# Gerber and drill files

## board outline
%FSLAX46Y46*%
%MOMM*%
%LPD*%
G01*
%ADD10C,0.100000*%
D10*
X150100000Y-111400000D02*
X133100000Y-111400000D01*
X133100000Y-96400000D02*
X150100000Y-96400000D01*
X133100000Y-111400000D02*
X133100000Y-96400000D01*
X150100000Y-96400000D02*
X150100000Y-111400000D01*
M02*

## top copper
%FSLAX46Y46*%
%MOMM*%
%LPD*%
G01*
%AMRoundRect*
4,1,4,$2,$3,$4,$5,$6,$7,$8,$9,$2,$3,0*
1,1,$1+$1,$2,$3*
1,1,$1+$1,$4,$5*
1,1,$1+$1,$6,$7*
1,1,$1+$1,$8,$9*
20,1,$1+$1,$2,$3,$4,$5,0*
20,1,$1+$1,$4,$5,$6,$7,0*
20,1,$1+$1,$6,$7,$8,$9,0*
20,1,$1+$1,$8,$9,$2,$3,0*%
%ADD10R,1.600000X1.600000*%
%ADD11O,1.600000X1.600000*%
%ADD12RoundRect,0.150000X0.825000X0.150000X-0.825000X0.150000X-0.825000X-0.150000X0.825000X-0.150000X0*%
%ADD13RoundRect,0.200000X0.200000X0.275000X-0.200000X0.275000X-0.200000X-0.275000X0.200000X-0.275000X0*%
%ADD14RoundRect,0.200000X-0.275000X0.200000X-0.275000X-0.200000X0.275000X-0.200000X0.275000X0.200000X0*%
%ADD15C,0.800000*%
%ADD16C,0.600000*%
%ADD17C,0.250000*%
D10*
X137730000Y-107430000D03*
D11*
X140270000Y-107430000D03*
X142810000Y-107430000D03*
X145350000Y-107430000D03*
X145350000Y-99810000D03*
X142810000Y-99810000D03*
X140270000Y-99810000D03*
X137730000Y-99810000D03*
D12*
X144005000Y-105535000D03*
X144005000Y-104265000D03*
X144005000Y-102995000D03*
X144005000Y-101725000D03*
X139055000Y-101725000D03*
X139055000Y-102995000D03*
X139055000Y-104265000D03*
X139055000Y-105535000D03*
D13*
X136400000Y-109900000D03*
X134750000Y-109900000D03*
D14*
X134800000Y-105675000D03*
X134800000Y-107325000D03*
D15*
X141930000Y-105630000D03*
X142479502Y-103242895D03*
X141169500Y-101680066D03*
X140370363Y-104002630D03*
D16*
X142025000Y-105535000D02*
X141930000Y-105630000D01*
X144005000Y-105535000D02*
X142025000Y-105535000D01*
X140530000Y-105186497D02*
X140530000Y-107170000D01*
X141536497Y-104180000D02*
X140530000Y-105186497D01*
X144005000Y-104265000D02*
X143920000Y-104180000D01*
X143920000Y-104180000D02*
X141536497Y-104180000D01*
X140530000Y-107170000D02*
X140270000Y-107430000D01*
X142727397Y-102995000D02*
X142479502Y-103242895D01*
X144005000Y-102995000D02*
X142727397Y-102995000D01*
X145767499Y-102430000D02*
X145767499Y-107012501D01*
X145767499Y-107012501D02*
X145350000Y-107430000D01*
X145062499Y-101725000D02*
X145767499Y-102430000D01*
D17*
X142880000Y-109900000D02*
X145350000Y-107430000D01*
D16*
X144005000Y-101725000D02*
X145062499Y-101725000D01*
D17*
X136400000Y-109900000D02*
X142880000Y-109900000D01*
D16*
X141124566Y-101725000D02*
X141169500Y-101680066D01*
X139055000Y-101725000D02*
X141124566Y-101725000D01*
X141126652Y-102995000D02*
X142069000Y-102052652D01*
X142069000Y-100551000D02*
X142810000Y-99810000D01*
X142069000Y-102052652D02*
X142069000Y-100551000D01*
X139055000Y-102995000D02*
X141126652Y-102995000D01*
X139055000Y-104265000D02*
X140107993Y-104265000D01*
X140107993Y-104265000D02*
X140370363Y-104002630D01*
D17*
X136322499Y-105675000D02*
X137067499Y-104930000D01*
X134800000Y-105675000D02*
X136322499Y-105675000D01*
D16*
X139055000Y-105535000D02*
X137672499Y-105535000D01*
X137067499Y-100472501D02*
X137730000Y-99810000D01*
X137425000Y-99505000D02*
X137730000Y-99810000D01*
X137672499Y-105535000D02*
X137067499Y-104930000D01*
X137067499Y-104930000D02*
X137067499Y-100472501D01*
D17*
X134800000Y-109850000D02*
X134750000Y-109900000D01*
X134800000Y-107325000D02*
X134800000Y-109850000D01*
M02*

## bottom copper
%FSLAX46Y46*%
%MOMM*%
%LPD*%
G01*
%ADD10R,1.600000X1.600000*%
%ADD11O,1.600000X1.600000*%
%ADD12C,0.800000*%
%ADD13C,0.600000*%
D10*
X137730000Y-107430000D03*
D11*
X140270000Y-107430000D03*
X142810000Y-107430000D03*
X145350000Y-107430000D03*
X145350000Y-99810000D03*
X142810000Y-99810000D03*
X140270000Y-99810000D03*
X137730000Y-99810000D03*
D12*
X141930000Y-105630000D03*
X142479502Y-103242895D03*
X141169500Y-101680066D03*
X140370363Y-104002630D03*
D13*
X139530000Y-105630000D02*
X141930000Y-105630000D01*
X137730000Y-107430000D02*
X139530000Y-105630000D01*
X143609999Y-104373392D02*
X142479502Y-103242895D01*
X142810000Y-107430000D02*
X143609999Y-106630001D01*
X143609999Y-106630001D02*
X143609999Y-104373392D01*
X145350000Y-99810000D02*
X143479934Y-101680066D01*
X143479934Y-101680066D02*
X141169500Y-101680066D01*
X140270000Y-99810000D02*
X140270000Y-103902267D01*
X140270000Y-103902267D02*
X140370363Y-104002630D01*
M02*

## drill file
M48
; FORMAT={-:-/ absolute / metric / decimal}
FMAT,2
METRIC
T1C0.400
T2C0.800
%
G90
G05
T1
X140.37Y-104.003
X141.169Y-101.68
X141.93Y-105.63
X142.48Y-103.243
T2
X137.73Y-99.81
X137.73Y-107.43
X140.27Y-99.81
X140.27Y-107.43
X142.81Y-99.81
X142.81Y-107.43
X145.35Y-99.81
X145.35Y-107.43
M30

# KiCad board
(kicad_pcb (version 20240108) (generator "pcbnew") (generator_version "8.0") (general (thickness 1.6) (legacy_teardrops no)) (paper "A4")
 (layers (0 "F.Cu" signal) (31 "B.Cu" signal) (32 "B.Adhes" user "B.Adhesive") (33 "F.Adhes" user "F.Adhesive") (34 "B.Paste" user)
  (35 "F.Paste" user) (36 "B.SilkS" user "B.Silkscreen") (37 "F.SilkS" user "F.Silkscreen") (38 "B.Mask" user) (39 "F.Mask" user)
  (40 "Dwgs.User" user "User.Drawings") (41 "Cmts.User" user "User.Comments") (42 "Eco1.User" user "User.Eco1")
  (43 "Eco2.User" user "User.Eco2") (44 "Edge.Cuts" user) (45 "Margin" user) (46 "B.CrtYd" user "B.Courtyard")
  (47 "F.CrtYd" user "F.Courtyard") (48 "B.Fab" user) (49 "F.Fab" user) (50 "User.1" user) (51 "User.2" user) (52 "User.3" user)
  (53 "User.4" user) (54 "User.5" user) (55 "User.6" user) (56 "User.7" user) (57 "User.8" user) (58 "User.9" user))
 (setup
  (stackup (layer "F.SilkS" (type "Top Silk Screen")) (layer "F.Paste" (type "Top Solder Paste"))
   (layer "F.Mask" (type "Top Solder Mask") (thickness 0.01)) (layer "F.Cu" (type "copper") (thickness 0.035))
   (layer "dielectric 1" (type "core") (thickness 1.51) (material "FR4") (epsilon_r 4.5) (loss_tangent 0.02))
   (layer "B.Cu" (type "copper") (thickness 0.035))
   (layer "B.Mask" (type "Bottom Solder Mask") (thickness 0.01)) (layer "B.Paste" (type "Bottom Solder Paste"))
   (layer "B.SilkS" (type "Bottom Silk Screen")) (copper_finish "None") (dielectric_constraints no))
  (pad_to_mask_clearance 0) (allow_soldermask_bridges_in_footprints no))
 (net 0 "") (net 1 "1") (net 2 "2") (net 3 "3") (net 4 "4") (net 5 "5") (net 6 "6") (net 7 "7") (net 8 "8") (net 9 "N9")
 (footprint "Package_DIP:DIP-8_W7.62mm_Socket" (layer "F.Cu") (at 137.73 107.43 90)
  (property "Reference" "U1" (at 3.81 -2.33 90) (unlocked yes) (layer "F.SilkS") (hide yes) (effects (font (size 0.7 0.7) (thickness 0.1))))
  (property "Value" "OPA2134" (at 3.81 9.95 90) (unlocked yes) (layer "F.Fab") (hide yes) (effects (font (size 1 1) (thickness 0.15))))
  (pad "1" thru_hole rect (at 0 0 90) (size 1.6 1.6) (drill 0.8) (layers "*.Cu" "*.Mask") (remove_unused_layers no) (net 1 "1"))
  (pad "2" thru_hole oval (at 0 2.54 90) (size 1.6 1.6) (drill 0.8) (layers "*.Cu" "*.Mask") (remove_unused_layers no) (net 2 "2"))
  (pad "3" thru_hole oval (at 0 5.08 90) (size 1.6 1.6) (drill 0.8) (layers "*.Cu" "*.Mask") (remove_unused_layers no) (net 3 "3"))
  (pad "4" thru_hole oval (at 0 7.62 90) (size 1.6 1.6) (drill 0.8) (layers "*.Cu" "*.Mask") (remove_unused_layers no) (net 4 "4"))
  (pad "5" thru_hole oval (at 7.62 7.62 90) (size 1.6 1.6) (drill 0.8) (layers "*.Cu" "*.Mask") (remove_unused_layers no) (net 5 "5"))
  (pad "6" thru_hole oval (at 7.62 5.08 90) (size 1.6 1.6) (drill 0.8) (layers "*.Cu" "*.Mask") (remove_unused_layers no) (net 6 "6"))
  (pad "7" thru_hole oval (at 7.62 2.54 90) (size 1.6 1.6) (drill 0.8) (layers "*.Cu" "*.Mask") (remove_unused_layers no) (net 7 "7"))
  (pad "8" thru_hole oval (at 7.62 0 90) (size 1.6 1.6) (drill 0.8) (layers "*.Cu" "*.Mask") (remove_unused_layers no) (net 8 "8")))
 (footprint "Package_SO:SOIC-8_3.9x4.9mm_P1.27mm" (layer "F.Cu") (at 141.53 103.63 180)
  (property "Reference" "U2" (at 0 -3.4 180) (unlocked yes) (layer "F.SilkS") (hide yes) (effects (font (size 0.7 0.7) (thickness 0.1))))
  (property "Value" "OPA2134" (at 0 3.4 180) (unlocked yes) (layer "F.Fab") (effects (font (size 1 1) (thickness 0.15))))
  (pad "1" smd roundrect (at -2.475 -1.905 180) (size 1.95 0.6) (layers "F.Cu" "F.Paste" "F.Mask") (roundrect_rratio 0.25) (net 1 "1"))
  (pad "2" smd roundrect (at -2.475 -0.635 180) (size 1.95 0.6) (layers "F.Cu" "F.Paste" "F.Mask") (roundrect_rratio 0.25) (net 2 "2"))
  (pad "3" smd roundrect (at -2.475 0.635 180) (size 1.95 0.6) (layers "F.Cu" "F.Paste" "F.Mask") (roundrect_rratio 0.25) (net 3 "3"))
  (pad "4" smd roundrect (at -2.475 1.905 180) (size 1.95 0.6) (layers "F.Cu" "F.Paste" "F.Mask") (roundrect_rratio 0.25) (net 4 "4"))
  (pad "5" smd roundrect (at 2.475 1.905 180) (size 1.95 0.6) (layers "F.Cu" "F.Paste" "F.Mask") (roundrect_rratio 0.25) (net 5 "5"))
  (pad "6" smd roundrect (at 2.475 0.635 180) (size 1.95 0.6) (layers "F.Cu" "F.Paste" "F.Mask") (roundrect_rratio 0.25) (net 6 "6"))
  (pad "7" smd roundrect (at 2.475 -0.635 180) (size 1.95 0.6) (layers "F.Cu" "F.Paste" "F.Mask") (roundrect_rratio 0.25) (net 7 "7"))
  (pad "8" smd roundrect (at 2.475 -1.905 180) (size 1.95 0.6) (layers "F.Cu" "F.Paste" "F.Mask") (roundrect_rratio 0.25) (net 8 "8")))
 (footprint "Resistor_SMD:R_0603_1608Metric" (layer "F.Cu") (at 135.575 109.9 180)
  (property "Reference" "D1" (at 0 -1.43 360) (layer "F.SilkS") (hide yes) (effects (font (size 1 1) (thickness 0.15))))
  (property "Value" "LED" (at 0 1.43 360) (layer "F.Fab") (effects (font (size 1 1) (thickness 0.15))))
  (pad "1" smd roundrect (at -0.825 0 180) (size 0.8 0.95) (layers "F.Cu" "F.Paste" "F.Mask") (roundrect_rratio 0.25) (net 4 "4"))
  (pad "2" smd roundrect (at 0.825 0 180) (size 0.8 0.95) (layers "F.Cu" "F.Paste" "F.Mask") (roundrect_rratio 0.25) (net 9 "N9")))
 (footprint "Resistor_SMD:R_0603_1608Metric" (layer "F.Cu") (at 134.8 106.5 -90)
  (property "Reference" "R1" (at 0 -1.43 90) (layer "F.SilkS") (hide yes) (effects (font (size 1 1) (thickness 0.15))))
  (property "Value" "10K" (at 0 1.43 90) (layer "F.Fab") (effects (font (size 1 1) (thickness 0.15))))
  (pad "1" smd roundrect (at -0.825 0 270) (size 0.8 0.95) (layers "F.Cu" "F.Paste" "F.Mask") (roundrect_rratio 0.25) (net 8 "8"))
  (pad "2" smd roundrect (at 0.825 0 270) (size 0.8 0.95) (layers "F.Cu" "F.Paste" "F.Mask") (roundrect_rratio 0.25) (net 9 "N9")))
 (gr_line (start 150.1 111.4) (end 133.1 111.4) (stroke (width 0.1) (type default)) (layer "Edge.Cuts"))
 (gr_line (start 133.1 96.4) (end 150.1 96.4) (stroke (width 0.1) (type default)) (layer "Edge.Cuts"))
 (gr_line (start 133.1 111.4) (end 133.1 96.4) (stroke (width 0.1) (type default)) (layer "Edge.Cuts"))
 (gr_line (start 150.1 96.4) (end 150.1 111.4) (stroke (width 0.1) (type default)) (layer "Edge.Cuts"))
 (segment (start 142.025 105.535) (end 141.93 105.63) (width 0.6) (layer "F.Cu") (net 1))
 (segment (start 144.005 105.535) (end 142.025 105.535) (width 0.6) (layer "F.Cu") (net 1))
 (via (at 141.93 105.63) (size 0.8) (drill 0.4) (layers "F.Cu" "B.Cu") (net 1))
 (segment (start 139.53 105.63) (end 141.93 105.63) (width 0.6) (layer "B.Cu") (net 1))
 (segment (start 137.73 107.43) (end 139.53 105.63) (width 0.6) (layer "B.Cu") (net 1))
 (segment (start 140.53 105.186497) (end 140.53 107.17) (width 0.6) (layer "F.Cu") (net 2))
 (segment (start 141.536497 104.18) (end 140.53 105.186497) (width 0.6) (layer "F.Cu") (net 2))
 (segment (start 144.005 104.265) (end 143.92 104.18) (width 0.6) (layer "F.Cu") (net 2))
 (segment (start 143.92 104.18) (end 141.536497 104.18) (width 0.6) (layer "F.Cu") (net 2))
 (segment (start 140.53 107.17) (end 140.27 107.43) (width 0.6) (layer "F.Cu") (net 2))
 (segment (start 142.727397 102.995) (end 142.479502 103.242895) (width 0.6) (layer "F.Cu") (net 3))
 (segment (start 144.005 102.995) (end 142.727397 102.995) (width 0.6) (layer "F.Cu") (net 3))
 (via (at 142.479502 103.242895) (size 0.8) (drill 0.4) (layers "F.Cu" "B.Cu") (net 3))
 (segment (start 143.609999 104.373392) (end 142.479502 103.242895) (width 0.6) (layer "B.Cu") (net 3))
 (segment (start 142.81 107.43) (end 143.609999 106.630001) (width 0.6) (layer "B.Cu") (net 3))
 (segment (start 143.609999 106.630001) (end 143.609999 104.373392) (width 0.6) (layer "B.Cu") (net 3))
 (segment (start 145.767499 102.43) (end 145.767499 107.012501) (width 0.6) (layer "F.Cu") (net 4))
 (segment (start 145.767499 107.012501) (end 145.35 107.43) (width 0.6) (layer "F.Cu") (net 4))
 (segment (start 145.062499 101.725) (end 145.767499 102.43) (width 0.6) (layer "F.Cu") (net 4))
 (segment (start 142.88 109.9) (end 145.35 107.43) (width 0.25) (layer "F.Cu") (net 4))
 (segment (start 144.005 101.725) (end 145.062499 101.725) (width 0.6) (layer "F.Cu") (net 4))
 (segment (start 136.4 109.9) (end 142.88 109.9) (width 0.25) (layer "F.Cu") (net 4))
 (segment (start 141.124566 101.725) (end 141.1695 101.680066) (width 0.6) (layer "F.Cu") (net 5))
 (segment (start 139.055 101.725) (end 141.124566 101.725) (width 0.6) (layer "F.Cu") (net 5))
 (via (at 141.1695 101.680066) (size 0.8) (drill 0.4) (layers "F.Cu" "B.Cu") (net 5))
 (segment (start 145.35 99.81) (end 143.479934 101.680066) (width 0.6) (layer "B.Cu") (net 5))
 (segment (start 143.479934 101.680066) (end 141.1695 101.680066) (width 0.6) (layer "B.Cu") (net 5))
 (segment (start 141.126652 102.995) (end 142.069 102.052652) (width 0.6) (layer "F.Cu") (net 6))
 (segment (start 142.069 100.551) (end 142.81 99.81) (width 0.6) (layer "F.Cu") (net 6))
 (segment (start 142.069 102.052652) (end 142.069 100.551) (width 0.6) (layer "F.Cu") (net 6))
 (segment (start 139.055 102.995) (end 141.126652 102.995) (width 0.6) (layer "F.Cu") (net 6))
 (segment (start 139.055 104.265) (end 140.107993 104.265) (width 0.6) (layer "F.Cu") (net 7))
 (segment (start 140.107993 104.265) (end 140.370363 104.00263) (width 0.6) (layer "F.Cu") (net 7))
 (via (at 140.370363 104.00263) (size 0.8) (drill 0.4) (layers "F.Cu" "B.Cu") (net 7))
 (segment (start 140.27 99.81) (end 140.27 103.902267) (width 0.6) (layer "B.Cu") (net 7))
 (segment (start 140.27 103.902267) (end 140.370363 104.00263) (width 0.6) (layer "B.Cu") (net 7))
 (segment (start 136.322499 105.675) (end 137.067499 104.93) (width 0.25) (layer "F.Cu") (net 8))
 (segment (start 134.8 105.675) (end 136.322499 105.675) (width 0.25) (layer "F.Cu") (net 8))
 (segment (start 139.055 105.535) (end 137.672499 105.535) (width 0.6) (layer "F.Cu") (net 8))
 (segment (start 137.067499 100.472501) (end 137.73 99.81) (width 0.6) (layer "F.Cu") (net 8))
 (segment (start 137.425 99.505) (end 137.73 99.81) (width 0.6) (layer "F.Cu") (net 8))
 (segment (start 137.672499 105.535) (end 137.067499 104.93) (width 0.6) (layer "F.Cu") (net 8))
 (segment (start 137.067499 104.93) (end 137.067499 100.472501) (width 0.6) (layer "F.Cu") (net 8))
 (segment (start 134.8 109.85) (end 134.75 109.9) (width 0.25) (layer "F.Cu") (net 9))
 (segment (start 134.8 107.325) (end 134.8 109.85) (width 0.25) (layer "F.Cu") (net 9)))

